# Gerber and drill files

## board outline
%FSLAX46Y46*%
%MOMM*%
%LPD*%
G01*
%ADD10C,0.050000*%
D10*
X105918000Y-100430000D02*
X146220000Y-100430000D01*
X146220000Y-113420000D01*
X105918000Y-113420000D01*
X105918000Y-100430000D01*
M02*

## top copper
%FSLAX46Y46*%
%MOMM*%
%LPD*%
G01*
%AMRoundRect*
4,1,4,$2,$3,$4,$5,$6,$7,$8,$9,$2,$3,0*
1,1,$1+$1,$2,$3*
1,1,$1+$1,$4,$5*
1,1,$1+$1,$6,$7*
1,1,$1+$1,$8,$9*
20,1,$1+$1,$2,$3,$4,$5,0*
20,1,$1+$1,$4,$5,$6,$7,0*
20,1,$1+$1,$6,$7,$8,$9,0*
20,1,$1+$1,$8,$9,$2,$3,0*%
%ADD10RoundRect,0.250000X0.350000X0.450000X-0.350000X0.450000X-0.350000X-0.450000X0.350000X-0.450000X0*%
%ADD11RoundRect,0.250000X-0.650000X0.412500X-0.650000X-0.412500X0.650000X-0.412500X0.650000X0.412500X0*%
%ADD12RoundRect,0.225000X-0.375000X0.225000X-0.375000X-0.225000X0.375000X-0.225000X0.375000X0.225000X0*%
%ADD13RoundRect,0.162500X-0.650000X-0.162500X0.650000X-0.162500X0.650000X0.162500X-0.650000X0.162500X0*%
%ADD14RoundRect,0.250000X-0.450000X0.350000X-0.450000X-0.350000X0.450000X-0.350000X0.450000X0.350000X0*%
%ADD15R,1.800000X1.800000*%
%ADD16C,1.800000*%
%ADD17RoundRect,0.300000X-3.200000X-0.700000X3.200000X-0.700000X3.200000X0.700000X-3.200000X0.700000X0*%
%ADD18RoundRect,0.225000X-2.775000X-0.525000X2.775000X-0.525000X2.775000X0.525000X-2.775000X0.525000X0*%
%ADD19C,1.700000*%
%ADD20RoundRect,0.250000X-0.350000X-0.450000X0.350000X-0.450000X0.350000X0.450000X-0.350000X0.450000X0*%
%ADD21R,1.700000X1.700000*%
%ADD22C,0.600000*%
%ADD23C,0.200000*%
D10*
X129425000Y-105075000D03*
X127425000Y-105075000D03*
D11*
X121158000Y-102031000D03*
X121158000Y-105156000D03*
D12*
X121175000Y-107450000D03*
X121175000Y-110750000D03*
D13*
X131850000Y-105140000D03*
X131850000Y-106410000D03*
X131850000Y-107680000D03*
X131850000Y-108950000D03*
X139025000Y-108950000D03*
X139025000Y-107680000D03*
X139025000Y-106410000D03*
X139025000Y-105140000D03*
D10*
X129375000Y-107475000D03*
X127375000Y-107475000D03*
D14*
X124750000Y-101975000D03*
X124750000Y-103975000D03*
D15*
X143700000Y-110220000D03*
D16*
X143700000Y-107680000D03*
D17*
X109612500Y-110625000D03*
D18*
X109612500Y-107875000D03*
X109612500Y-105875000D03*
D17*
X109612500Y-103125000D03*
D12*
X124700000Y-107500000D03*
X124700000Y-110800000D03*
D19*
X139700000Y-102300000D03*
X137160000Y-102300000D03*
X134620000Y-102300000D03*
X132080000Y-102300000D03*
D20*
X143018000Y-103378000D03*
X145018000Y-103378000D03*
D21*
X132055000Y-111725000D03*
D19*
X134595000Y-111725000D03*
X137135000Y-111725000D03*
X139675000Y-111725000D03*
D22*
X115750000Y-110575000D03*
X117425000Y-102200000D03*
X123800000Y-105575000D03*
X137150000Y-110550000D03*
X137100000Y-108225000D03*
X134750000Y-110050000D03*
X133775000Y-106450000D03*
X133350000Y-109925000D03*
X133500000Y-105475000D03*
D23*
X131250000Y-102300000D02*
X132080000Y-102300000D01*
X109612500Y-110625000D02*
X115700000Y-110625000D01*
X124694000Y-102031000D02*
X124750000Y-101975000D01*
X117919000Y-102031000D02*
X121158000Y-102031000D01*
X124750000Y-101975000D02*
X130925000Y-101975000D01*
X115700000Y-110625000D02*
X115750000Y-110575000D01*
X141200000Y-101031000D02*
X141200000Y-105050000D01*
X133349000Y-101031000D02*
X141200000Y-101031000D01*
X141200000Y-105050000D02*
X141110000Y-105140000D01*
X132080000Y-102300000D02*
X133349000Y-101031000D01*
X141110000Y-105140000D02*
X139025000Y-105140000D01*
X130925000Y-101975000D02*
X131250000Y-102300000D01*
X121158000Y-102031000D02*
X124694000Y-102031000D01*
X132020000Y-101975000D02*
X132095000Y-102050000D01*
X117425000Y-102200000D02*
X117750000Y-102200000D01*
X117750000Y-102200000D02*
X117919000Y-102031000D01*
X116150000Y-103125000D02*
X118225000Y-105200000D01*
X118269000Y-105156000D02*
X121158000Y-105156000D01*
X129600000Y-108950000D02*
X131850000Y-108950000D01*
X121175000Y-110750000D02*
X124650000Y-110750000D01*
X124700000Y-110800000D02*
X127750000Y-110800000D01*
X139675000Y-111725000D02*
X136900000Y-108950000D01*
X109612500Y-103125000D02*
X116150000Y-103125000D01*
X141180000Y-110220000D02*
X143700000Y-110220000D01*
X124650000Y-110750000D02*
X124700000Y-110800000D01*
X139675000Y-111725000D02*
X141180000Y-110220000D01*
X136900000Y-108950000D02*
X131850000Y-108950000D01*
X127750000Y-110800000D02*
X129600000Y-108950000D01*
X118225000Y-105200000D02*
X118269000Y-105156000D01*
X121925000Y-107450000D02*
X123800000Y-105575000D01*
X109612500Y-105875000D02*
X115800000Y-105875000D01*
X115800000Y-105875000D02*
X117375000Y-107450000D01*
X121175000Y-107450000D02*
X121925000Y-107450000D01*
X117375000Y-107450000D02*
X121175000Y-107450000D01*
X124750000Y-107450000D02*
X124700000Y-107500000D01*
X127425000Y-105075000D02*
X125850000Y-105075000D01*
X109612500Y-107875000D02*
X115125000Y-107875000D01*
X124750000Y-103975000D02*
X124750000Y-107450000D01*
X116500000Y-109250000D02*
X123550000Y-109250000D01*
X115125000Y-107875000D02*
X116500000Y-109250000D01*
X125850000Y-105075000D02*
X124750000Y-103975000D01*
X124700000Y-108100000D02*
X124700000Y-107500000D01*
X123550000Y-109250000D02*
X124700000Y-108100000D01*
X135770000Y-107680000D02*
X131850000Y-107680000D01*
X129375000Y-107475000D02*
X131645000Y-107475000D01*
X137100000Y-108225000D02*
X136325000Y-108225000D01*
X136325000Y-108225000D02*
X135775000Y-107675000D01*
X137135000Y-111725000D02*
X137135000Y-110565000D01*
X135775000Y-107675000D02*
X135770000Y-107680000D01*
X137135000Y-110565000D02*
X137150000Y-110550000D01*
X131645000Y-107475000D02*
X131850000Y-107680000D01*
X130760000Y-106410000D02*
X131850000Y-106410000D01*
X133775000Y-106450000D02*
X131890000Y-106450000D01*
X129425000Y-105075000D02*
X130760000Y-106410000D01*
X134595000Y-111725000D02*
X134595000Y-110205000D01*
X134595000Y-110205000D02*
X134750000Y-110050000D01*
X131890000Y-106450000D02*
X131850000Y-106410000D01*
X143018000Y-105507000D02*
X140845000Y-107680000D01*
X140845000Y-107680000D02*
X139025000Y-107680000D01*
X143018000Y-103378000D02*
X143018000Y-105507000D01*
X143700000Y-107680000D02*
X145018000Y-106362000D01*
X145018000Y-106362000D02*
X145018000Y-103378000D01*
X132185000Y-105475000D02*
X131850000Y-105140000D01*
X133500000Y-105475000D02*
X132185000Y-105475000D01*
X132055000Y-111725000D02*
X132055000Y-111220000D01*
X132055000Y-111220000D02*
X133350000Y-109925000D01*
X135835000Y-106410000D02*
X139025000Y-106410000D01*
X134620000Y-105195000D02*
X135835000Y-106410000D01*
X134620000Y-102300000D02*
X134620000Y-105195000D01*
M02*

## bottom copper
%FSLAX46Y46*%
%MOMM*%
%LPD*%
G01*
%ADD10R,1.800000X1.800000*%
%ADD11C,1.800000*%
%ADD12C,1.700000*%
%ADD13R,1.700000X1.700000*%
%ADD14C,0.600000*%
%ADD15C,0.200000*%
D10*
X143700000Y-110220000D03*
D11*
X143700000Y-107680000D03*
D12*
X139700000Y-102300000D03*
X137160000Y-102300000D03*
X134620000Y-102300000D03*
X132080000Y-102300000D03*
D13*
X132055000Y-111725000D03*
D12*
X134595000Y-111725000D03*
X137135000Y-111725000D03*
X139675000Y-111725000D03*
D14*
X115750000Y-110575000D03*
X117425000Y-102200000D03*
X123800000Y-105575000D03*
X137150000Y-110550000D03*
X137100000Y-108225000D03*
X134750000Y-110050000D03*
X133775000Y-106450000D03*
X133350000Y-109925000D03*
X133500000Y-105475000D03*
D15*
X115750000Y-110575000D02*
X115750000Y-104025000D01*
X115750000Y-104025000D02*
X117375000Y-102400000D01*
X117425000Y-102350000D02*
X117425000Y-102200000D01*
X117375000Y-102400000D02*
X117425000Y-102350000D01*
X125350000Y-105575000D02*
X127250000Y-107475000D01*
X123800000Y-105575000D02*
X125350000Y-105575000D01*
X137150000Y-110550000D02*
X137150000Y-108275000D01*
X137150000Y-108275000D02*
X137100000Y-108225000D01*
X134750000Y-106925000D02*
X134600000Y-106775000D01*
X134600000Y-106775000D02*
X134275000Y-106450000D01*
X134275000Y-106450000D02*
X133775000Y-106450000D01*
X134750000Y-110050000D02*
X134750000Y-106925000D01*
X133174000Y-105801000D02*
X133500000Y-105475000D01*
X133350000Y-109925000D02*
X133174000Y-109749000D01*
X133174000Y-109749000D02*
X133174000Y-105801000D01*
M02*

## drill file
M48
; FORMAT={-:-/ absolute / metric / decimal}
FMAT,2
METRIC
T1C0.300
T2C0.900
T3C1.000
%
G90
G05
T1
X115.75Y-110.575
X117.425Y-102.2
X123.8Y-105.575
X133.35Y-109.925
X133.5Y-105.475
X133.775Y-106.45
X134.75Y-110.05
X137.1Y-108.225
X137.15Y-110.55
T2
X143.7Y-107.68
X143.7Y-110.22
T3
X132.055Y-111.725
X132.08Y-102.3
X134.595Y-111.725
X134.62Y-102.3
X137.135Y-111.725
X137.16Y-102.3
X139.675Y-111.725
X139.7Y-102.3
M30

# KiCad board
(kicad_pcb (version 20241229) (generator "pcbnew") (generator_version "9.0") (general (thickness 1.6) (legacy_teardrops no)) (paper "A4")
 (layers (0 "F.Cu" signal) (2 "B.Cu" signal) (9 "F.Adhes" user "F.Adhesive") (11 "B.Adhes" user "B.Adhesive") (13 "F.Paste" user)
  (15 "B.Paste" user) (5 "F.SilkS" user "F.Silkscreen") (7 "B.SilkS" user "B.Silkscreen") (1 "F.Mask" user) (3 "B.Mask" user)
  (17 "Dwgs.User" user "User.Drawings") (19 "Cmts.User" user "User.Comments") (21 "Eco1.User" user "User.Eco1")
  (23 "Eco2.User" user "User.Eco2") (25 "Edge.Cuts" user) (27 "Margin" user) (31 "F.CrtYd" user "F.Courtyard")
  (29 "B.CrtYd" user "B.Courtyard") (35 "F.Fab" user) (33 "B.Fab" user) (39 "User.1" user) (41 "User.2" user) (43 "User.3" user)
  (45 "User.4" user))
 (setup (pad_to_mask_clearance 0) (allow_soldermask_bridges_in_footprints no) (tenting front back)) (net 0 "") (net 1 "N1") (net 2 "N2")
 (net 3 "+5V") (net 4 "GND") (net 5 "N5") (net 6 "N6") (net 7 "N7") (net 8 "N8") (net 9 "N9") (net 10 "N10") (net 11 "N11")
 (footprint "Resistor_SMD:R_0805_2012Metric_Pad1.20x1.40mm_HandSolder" (layer "F.Cu") (at 128.425 105.075 180)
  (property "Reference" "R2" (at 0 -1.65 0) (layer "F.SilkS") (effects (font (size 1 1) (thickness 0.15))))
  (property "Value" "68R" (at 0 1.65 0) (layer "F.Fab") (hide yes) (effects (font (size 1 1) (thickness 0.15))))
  (pad "1" smd roundrect (at -1 0 180) (size 1.2 1.4) (layers "F.Cu" "F.Mask" "F.Paste") (roundrect_rratio 0.208333) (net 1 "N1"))
  (pad "2" smd roundrect (at 1 0 180) (size 1.2 1.4) (layers "F.Cu" "F.Mask" "F.Paste") (roundrect_rratio 0.208333) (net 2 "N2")))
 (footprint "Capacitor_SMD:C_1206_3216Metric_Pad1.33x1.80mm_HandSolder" (layer "F.Cu") (at 121.158 103.5935 -90)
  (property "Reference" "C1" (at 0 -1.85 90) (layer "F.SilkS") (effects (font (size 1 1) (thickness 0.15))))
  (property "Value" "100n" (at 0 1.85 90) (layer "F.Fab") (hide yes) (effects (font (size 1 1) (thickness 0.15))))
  (pad "1" smd roundrect (at -1.5625 0 270) (size 1.325 1.8) (layers "F.Cu" "F.Mask" "F.Paste") (roundrect_rratio 0.188679) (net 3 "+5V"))
  (pad "2" smd roundrect (at 1.5625 0 270) (size 1.325 1.8) (layers "F.Cu" "F.Mask" "F.Paste") (roundrect_rratio 0.188679) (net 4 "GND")))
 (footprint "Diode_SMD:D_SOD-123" (layer "F.Cu") (at 121.175 109.1 -90)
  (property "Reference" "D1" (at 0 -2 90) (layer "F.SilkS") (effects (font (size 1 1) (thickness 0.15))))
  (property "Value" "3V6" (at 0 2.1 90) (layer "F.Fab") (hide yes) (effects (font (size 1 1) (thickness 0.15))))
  (pad "1" smd roundrect (at -1.65 0 270) (size 0.9 1.2) (layers "F.Cu" "F.Mask" "F.Paste") (roundrect_rratio 0.25) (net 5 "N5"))
  (pad "2" smd roundrect (at 1.65 0 270) (size 0.9 1.2) (layers "F.Cu" "F.Mask" "F.Paste") (roundrect_rratio 0.25) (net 4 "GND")))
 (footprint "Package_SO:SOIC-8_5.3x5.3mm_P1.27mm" (layer "F.Cu") (at 135.4375 107.045)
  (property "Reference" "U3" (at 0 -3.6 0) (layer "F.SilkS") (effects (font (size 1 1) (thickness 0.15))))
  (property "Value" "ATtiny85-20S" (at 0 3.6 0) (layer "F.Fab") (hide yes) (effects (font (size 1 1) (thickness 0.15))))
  (pad "1" smd roundrect (at -3.5875 -1.905) (size 1.625 0.65) (layers "F.Cu" "F.Mask" "F.Paste") (roundrect_rratio 0.25) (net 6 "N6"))
  (pad "2" smd roundrect (at -3.5875 -0.635) (size 1.625 0.65) (layers "F.Cu" "F.Mask" "F.Paste") (roundrect_rratio 0.25) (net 1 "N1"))
  (pad "3" smd roundrect (at -3.5875 0.635) (size 1.625 0.65) (layers "F.Cu" "F.Mask" "F.Paste") (roundrect_rratio 0.25) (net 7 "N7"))
  (pad "4" smd roundrect (at -3.5875 1.905) (size 1.625 0.65) (layers "F.Cu" "F.Mask" "F.Paste") (roundrect_rratio 0.25) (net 4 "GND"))
  (pad "5" smd roundrect (at 3.5875 1.905) (size 1.625 0.65) (layers "F.Cu" "F.Mask" "F.Paste") (roundrect_rratio 0.25) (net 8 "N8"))
  (pad "6" smd roundrect (at 3.5875 0.635) (size 1.625 0.65) (layers "F.Cu" "F.Mask" "F.Paste") (roundrect_rratio 0.25) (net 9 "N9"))
  (pad "7" smd roundrect (at 3.5875 -0.635) (size 1.625 0.65) (layers "F.Cu" "F.Mask" "F.Paste") (roundrect_rratio 0.25) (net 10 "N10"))
  (pad "8" smd roundrect (at 3.5875 -1.905) (size 1.625 0.65) (layers "F.Cu" "F.Mask" "F.Paste") (roundrect_rratio 0.25) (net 3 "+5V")))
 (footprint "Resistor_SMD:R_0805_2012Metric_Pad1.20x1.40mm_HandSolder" (layer "F.Cu") (at 128.375 107.475 180)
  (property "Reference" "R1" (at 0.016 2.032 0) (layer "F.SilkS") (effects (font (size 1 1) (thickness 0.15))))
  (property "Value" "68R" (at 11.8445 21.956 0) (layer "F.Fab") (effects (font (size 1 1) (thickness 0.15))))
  (pad "1" smd roundrect (at -1 0 180) (size 1.2 1.4) (layers "F.Cu" "F.Mask" "F.Paste") (roundrect_rratio 0.208333) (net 7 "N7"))
  (pad "2" smd roundrect (at 1 0 180) (size 1.2 1.4) (layers "F.Cu" "F.Mask" "F.Paste") (roundrect_rratio 0.208333) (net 5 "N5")))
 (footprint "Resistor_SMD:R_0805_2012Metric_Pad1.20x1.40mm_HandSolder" (layer "F.Cu") (at 124.75 102.975 -90)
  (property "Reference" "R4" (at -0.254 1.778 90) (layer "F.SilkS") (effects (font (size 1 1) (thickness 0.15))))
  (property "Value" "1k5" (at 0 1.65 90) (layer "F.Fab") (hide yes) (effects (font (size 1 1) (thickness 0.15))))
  (pad "1" smd roundrect (at -1 0 270) (size 1.2 1.4) (layers "F.Cu" "F.Mask" "F.Paste") (roundrect_rratio 0.208333) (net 3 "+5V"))
  (pad "2" smd roundrect (at 1 0 270) (size 1.2 1.4) (layers "F.Cu" "F.Mask" "F.Paste") (roundrect_rratio 0.208333) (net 2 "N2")))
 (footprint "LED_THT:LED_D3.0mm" (layer "F.Cu") (at 143.7 110.22 90)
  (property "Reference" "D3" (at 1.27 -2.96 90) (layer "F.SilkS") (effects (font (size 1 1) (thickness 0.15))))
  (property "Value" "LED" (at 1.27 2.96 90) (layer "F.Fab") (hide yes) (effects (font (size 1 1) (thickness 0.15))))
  (pad "1" thru_hole rect (at 0 0 90) (size 1.8 1.8) (drill 0.9) (layers "*.Cu" "*.Mask") (remove_unused_layers no) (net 4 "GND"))
  (pad "2" thru_hole circle (at 2.54 0 90) (size 1.8 1.8) (drill 0.9) (layers "*.Cu" "*.Mask") (remove_unused_layers no) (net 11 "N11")))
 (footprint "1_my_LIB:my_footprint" (layer "F.Cu") (at 109.6125 106.875)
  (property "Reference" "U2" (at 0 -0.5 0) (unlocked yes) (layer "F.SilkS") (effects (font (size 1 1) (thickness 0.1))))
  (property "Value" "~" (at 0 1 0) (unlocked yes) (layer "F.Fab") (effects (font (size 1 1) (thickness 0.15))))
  (pad "1" smd roundrect (at 0 3.75) (size 7 2) (layers "F.Cu" "F.Mask" "F.Paste") (roundrect_rratio 0.15) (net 3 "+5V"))
  (pad "2" smd roundrect (at 0 1) (size 6 1.5) (layers "F.Cu" "F.Mask" "F.Paste") (roundrect_rratio 0.15) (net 2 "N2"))
  (pad "3" smd roundrect (at 0 -1) (size 6 1.5) (layers "F.Cu" "F.Mask" "F.Paste") (roundrect_rratio 0.15) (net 5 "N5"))
  (pad "4" smd roundrect (at 0 -3.75) (size 7 2) (layers "F.Cu" "F.Mask" "F.Paste") (roundrect_rratio 0.15) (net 4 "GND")))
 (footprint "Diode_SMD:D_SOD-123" (layer "F.Cu") (at 124.7 109.15 -90)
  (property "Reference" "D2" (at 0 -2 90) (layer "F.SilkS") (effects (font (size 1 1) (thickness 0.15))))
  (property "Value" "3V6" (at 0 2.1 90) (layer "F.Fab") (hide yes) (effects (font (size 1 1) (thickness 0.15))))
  (pad "1" smd roundrect (at -1.65 0 270) (size 0.9 1.2) (layers "F.Cu" "F.Mask" "F.Paste") (roundrect_rratio 0.25) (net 2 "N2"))
  (pad "2" smd roundrect (at 1.65 0 270) (size 0.9 1.2) (layers "F.Cu" "F.Mask" "F.Paste") (roundrect_rratio 0.25) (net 4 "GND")))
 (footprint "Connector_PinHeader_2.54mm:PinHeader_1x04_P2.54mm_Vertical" (layer "F.Cu") (at 139.7 102.3 -90)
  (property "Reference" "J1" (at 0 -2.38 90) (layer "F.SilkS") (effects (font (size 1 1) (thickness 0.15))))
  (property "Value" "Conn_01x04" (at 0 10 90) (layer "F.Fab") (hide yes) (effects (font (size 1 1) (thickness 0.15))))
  (pad "1" thru_hole circle (at 0 0 270) (size 1.7 1.7) (drill 1) (layers "*.Cu" "*.Mask") (remove_unused_layers no) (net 8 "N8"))
  (pad "2" thru_hole circle (at 0 2.54 270) (size 1.7 1.7) (drill 1) (layers "*.Cu" "*.Mask") (remove_unused_layers no) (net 9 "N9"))
  (pad "3" thru_hole circle (at 0 5.08 270) (size 1.7 1.7) (drill 1) (layers "*.Cu" "*.Mask") (remove_unused_layers no) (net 10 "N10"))
  (pad "4" thru_hole circle (at 0 7.62 270) (size 1.7 1.7) (drill 1) (layers "*.Cu" "*.Mask") (remove_unused_layers no) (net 3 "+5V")))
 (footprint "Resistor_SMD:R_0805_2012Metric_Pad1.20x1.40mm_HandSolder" (layer "F.Cu") (at 144.018 103.378)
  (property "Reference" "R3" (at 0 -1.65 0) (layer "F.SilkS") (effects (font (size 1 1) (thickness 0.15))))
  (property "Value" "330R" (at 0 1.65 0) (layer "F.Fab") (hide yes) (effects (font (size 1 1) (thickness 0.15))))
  (pad "1" smd roundrect (at -1 0) (size 1.2 1.4) (layers "F.Cu" "F.Mask" "F.Paste") (roundrect_rratio 0.208333) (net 9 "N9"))
  (pad "2" smd roundrect (at 1 0) (size 1.2 1.4) (layers "F.Cu" "F.Mask" "F.Paste") (roundrect_rratio 0.208333) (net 11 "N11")))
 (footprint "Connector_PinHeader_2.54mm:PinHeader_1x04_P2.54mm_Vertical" (layer "F.Cu") (at 132.055 111.725 90)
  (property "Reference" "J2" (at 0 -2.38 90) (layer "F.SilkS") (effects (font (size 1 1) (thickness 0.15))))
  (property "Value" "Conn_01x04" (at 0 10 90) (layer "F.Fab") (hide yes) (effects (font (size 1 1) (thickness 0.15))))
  (pad "1" thru_hole rect (at 0 0 90) (size 1.7 1.7) (drill 1) (layers "*.Cu" "*.Mask") (remove_unused_layers no) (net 6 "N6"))
  (pad "2" thru_hole circle (at 0 2.54 90) (size 1.7 1.7) (drill 1) (layers "*.Cu" "*.Mask") (remove_unused_layers no) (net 1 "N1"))
  (pad "3" thru_hole circle (at 0 5.08 90) (size 1.7 1.7) (drill 1) (layers "*.Cu" "*.Mask") (remove_unused_layers no) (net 7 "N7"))
  (pad "4" thru_hole circle (at 0 7.62 90) (size 1.7 1.7) (drill 1) (layers "*.Cu" "*.Mask") (remove_unused_layers no) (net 4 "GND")))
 (gr_rect (start 105.918 100.43) (end 146.22 113.42) (stroke (width 0.05) (type solid)) (fill no) (layer "Edge.Cuts"))
 (segment (start 131.25 102.3) (end 132.08 102.3) (width 0.2) (layer "F.Cu") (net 3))
 (segment (start 109.6125 110.625) (end 115.7 110.625) (width 0.2) (layer "F.Cu") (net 3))
 (segment (start 124.694 102.031) (end 124.75 101.975) (width 0.2) (layer "F.Cu") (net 3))
 (segment (start 117.919 102.031) (end 121.158 102.031) (width 0.2) (layer "F.Cu") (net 3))
 (segment (start 124.75 101.975) (end 130.925 101.975) (width 0.2) (layer "F.Cu") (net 3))
 (segment (start 115.7 110.625) (end 115.75 110.575) (width 0.2) (layer "F.Cu") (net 3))
 (segment (start 141.2 101.031) (end 141.2 105.05) (width 0.2) (layer "F.Cu") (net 3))
 (segment (start 133.349 101.031) (end 141.2 101.031) (width 0.2) (layer "F.Cu") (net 3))
 (segment (start 141.2 105.05) (end 141.11 105.14) (width 0.2) (layer "F.Cu") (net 3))
 (segment (start 132.08 102.3) (end 133.349 101.031) (width 0.2) (layer "F.Cu") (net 3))
 (segment (start 141.11 105.14) (end 139.025 105.14) (width 0.2) (layer "F.Cu") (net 3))
 (segment (start 130.925 101.975) (end 131.25 102.3) (width 0.2) (layer "F.Cu") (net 3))
 (segment (start 121.158 102.031) (end 124.694 102.031) (width 0.2) (layer "F.Cu") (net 3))
 (segment (start 132.02 101.975) (end 132.095 102.05) (width 0.2) (layer "F.Cu") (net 3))
 (segment (start 117.425 102.2) (end 117.75 102.2) (width 0.2) (layer "F.Cu") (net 3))
 (segment (start 117.75 102.2) (end 117.919 102.031) (width 0.2) (layer "F.Cu") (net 3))
 (via (at 115.75 110.575) (size 0.6) (drill 0.3) (layers "F.Cu" "B.Cu") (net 3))
 (via (at 117.425 102.2) (size 0.6) (drill 0.3) (layers "F.Cu" "B.Cu") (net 3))
 (segment (start 115.75 110.575) (end 115.75 104.025) (width 0.2) (layer "B.Cu") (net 3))
 (segment (start 115.75 104.025) (end 117.375 102.4) (width 0.2) (layer "B.Cu") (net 3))
 (segment (start 117.425 102.35) (end 117.425 102.2) (width 0.2) (layer "B.Cu") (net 3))
 (segment (start 117.375 102.4) (end 117.425 102.35) (width 0.2) (layer "B.Cu") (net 3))
 (segment (start 116.15 103.125) (end 118.225 105.2) (width 0.2) (layer "F.Cu") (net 4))
 (segment (start 118.269 105.156) (end 121.158 105.156) (width 0.2) (layer "F.Cu") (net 4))
 (segment (start 129.6 108.95) (end 131.85 108.95) (width 0.2) (layer "F.Cu") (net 4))
 (segment (start 121.175 110.75) (end 124.65 110.75) (width 0.2) (layer "F.Cu") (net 4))
 (segment (start 124.7 110.8) (end 127.75 110.8) (width 0.2) (layer "F.Cu") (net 4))
 (segment (start 139.675 111.725) (end 136.9 108.95) (width 0.2) (layer "F.Cu") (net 4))
 (segment (start 109.6125 103.125) (end 116.15 103.125) (width 0.2) (layer "F.Cu") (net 4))
 (segment (start 141.18 110.22) (end 143.7 110.22) (width 0.2) (layer "F.Cu") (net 4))
 (segment (start 124.65 110.75) (end 124.7 110.8) (width 0.2) (layer "F.Cu") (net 4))
 (segment (start 139.675 111.725) (end 141.18 110.22) (width 0.2) (layer "F.Cu") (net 4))
 (segment (start 136.9 108.95) (end 131.85 108.95) (width 0.2) (layer "F.Cu") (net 4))
 (segment (start 127.75 110.8) (end 129.6 108.95) (width 0.2) (layer "F.Cu") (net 4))
 (segment (start 118.225 105.2) (end 118.269 105.156) (width 0.2) (layer "F.Cu") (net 4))
 (segment (start 121.925 107.45) (end 123.8 105.575) (width 0.2) (layer "F.Cu") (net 5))
 (segment (start 109.6125 105.875) (end 115.8 105.875) (width 0.2) (layer "F.Cu") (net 5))
 (segment (start 115.8 105.875) (end 117.375 107.45) (width 0.2) (layer "F.Cu") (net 5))
 (segment (start 121.175 107.45) (end 121.925 107.45) (width 0.2) (layer "F.Cu") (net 5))
 (segment (start 117.375 107.45) (end 121.175 107.45) (width 0.2) (layer "F.Cu") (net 5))
 (via (at 123.8 105.575) (size 0.6) (drill 0.3) (layers "F.Cu" "B.Cu") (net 5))
 (segment (start 125.35 105.575) (end 127.25 107.475) (width 0.2) (layer "B.Cu") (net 5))
 (segment (start 123.8 105.575) (end 125.35 105.575) (width 0.2) (layer "B.Cu") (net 5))
 (segment (start 124.75 107.45) (end 124.7 107.5) (width 0.2) (layer "F.Cu") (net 2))
 (segment (start 127.425 105.075) (end 125.85 105.075) (width 0.2) (layer "F.Cu") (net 2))
 (segment (start 109.6125 107.875) (end 115.125 107.875) (width 0.2) (layer "F.Cu") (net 2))
 (segment (start 124.75 103.975) (end 124.75 107.45) (width 0.2) (layer "F.Cu") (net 2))
 (segment (start 116.5 109.25) (end 123.55 109.25) (width 0.2) (layer "F.Cu") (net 2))
 (segment (start 115.125 107.875) (end 116.5 109.25) (width 0.2) (layer "F.Cu") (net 2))
 (segment (start 125.85 105.075) (end 124.75 103.975) (width 0.2) (layer "F.Cu") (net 2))
 (segment (start 124.7 108.1) (end 124.7 107.5) (width 0.2) (layer "F.Cu") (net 2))
 (segment (start 123.55 109.25) (end 124.7 108.1) (width 0.2) (layer "F.Cu") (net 2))
 (segment (start 135.77 107.68) (end 131.85 107.68) (width 0.2) (layer "F.Cu") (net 7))
 (segment (start 129.375 107.475) (end 131.645 107.475) (width 0.2) (layer "F.Cu") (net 7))
 (segment (start 137.1 108.225) (end 136.325 108.225) (width 0.2) (layer "F.Cu") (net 7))
 (segment (start 136.325 108.225) (end 135.775 107.675) (width 0.2) (layer "F.Cu") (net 7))
 (segment (start 137.135 111.725) (end 137.135 110.565) (width 0.2) (layer "F.Cu") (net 7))
 (segment (start 135.775 107.675) (end 135.77 107.68) (width 0.2) (layer "F.Cu") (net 7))
 (segment (start 137.135 110.565) (end 137.15 110.55) (width 0.2) (layer "F.Cu") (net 7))
 (segment (start 131.645 107.475) (end 131.85 107.68) (width 0.2) (layer "F.Cu") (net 7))
 (via (at 137.15 110.55) (size 0.6) (drill 0.3) (layers "F.Cu" "B.Cu") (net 7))
 (via (at 137.1 108.225) (size 0.6) (drill 0.3) (layers "F.Cu" "B.Cu") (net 7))
 (segment (start 137.15 110.55) (end 137.15 108.275) (width 0.2) (layer "B.Cu") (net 7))
 (segment (start 137.15 108.275) (end 137.1 108.225) (width 0.2) (layer "B.Cu") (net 7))
 (segment (start 130.76 106.41) (end 131.85 106.41) (width 0.2) (layer "F.Cu") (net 1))
 (segment (start 133.775 106.45) (end 131.89 106.45) (width 0.2) (layer "F.Cu") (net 1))
 (segment (start 129.425 105.075) (end 130.76 106.41) (width 0.2) (layer "F.Cu") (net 1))
 (segment (start 134.595 111.725) (end 134.595 110.205) (width 0.2) (layer "F.Cu") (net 1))
 (segment (start 134.595 110.205) (end 134.75 110.05) (width 0.2) (layer "F.Cu") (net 1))
 (segment (start 131.89 106.45) (end 131.85 106.41) (width 0.2) (layer "F.Cu") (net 1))
 (via (at 134.75 110.05) (size 0.6) (drill 0.3) (layers "F.Cu" "B.Cu") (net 1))
 (via (at 133.775 106.45) (size 0.6) (drill 0.3) (layers "F.Cu" "B.Cu") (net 1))
 (segment (start 134.75 106.925) (end 134.6 106.775) (width 0.2) (layer "B.Cu") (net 1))
 (segment (start 134.6 106.775) (end 134.275 106.45) (width 0.2) (layer "B.Cu") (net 1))
 (segment (start 134.275 106.45) (end 133.775 106.45) (width 0.2) (layer "B.Cu") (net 1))
 (segment (start 134.75 110.05) (end 134.75 106.925) (width 0.2) (layer "B.Cu") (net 1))
 (segment (start 143.018 105.507) (end 140.845 107.68) (width 0.2) (layer "F.Cu") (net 9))
 (segment (start 140.845 107.68) (end 139.025 107.68) (width 0.2) (layer "F.Cu") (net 9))
 (segment (start 143.018 103.378) (end 143.018 105.507) (width 0.2) (layer "F.Cu") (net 9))
 (segment (start 143.7 107.68) (end 145.018 106.362) (width 0.2) (layer "F.Cu") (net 11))
 (segment (start 145.018 106.362) (end 145.018 103.378) (width 0.2) (layer "F.Cu") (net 11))
 (segment (start 132.185 105.475) (end 131.85 105.14) (width 0.2) (layer "F.Cu") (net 6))
 (segment (start 133.5 105.475) (end 132.185 105.475) (width 0.2) (layer "F.Cu") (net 6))
 (segment (start 132.055 111.725) (end 132.055 111.22) (width 0.2) (layer "F.Cu") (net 6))
 (segment (start 132.055 111.22) (end 133.35 109.925) (width 0.2) (layer "F.Cu") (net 6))
 (via (at 133.35 109.925) (size 0.6) (drill 0.3) (layers "F.Cu" "B.Cu") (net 6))
 (via (at 133.5 105.475) (size 0.6) (drill 0.3) (layers "F.Cu" "B.Cu") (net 6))
 (segment (start 133.174 105.801) (end 133.5 105.475) (width 0.2) (layer "B.Cu") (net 6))
 (segment (start 133.35 109.925) (end 133.174 109.749) (width 0.2) (layer "B.Cu") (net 6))
 (segment (start 133.174 109.749) (end 133.174 105.801) (width 0.2) (layer "B.Cu") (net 6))
 (segment (start 135.835 106.41) (end 139.025 106.41) (width 0.2) (layer "F.Cu") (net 10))
 (segment (start 134.62 105.195) (end 135.835 106.41) (width 0.2) (layer "F.Cu") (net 10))
 (segment (start 134.62 102.3) (end 134.62 105.195) (width 0.2) (layer "F.Cu") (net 10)))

